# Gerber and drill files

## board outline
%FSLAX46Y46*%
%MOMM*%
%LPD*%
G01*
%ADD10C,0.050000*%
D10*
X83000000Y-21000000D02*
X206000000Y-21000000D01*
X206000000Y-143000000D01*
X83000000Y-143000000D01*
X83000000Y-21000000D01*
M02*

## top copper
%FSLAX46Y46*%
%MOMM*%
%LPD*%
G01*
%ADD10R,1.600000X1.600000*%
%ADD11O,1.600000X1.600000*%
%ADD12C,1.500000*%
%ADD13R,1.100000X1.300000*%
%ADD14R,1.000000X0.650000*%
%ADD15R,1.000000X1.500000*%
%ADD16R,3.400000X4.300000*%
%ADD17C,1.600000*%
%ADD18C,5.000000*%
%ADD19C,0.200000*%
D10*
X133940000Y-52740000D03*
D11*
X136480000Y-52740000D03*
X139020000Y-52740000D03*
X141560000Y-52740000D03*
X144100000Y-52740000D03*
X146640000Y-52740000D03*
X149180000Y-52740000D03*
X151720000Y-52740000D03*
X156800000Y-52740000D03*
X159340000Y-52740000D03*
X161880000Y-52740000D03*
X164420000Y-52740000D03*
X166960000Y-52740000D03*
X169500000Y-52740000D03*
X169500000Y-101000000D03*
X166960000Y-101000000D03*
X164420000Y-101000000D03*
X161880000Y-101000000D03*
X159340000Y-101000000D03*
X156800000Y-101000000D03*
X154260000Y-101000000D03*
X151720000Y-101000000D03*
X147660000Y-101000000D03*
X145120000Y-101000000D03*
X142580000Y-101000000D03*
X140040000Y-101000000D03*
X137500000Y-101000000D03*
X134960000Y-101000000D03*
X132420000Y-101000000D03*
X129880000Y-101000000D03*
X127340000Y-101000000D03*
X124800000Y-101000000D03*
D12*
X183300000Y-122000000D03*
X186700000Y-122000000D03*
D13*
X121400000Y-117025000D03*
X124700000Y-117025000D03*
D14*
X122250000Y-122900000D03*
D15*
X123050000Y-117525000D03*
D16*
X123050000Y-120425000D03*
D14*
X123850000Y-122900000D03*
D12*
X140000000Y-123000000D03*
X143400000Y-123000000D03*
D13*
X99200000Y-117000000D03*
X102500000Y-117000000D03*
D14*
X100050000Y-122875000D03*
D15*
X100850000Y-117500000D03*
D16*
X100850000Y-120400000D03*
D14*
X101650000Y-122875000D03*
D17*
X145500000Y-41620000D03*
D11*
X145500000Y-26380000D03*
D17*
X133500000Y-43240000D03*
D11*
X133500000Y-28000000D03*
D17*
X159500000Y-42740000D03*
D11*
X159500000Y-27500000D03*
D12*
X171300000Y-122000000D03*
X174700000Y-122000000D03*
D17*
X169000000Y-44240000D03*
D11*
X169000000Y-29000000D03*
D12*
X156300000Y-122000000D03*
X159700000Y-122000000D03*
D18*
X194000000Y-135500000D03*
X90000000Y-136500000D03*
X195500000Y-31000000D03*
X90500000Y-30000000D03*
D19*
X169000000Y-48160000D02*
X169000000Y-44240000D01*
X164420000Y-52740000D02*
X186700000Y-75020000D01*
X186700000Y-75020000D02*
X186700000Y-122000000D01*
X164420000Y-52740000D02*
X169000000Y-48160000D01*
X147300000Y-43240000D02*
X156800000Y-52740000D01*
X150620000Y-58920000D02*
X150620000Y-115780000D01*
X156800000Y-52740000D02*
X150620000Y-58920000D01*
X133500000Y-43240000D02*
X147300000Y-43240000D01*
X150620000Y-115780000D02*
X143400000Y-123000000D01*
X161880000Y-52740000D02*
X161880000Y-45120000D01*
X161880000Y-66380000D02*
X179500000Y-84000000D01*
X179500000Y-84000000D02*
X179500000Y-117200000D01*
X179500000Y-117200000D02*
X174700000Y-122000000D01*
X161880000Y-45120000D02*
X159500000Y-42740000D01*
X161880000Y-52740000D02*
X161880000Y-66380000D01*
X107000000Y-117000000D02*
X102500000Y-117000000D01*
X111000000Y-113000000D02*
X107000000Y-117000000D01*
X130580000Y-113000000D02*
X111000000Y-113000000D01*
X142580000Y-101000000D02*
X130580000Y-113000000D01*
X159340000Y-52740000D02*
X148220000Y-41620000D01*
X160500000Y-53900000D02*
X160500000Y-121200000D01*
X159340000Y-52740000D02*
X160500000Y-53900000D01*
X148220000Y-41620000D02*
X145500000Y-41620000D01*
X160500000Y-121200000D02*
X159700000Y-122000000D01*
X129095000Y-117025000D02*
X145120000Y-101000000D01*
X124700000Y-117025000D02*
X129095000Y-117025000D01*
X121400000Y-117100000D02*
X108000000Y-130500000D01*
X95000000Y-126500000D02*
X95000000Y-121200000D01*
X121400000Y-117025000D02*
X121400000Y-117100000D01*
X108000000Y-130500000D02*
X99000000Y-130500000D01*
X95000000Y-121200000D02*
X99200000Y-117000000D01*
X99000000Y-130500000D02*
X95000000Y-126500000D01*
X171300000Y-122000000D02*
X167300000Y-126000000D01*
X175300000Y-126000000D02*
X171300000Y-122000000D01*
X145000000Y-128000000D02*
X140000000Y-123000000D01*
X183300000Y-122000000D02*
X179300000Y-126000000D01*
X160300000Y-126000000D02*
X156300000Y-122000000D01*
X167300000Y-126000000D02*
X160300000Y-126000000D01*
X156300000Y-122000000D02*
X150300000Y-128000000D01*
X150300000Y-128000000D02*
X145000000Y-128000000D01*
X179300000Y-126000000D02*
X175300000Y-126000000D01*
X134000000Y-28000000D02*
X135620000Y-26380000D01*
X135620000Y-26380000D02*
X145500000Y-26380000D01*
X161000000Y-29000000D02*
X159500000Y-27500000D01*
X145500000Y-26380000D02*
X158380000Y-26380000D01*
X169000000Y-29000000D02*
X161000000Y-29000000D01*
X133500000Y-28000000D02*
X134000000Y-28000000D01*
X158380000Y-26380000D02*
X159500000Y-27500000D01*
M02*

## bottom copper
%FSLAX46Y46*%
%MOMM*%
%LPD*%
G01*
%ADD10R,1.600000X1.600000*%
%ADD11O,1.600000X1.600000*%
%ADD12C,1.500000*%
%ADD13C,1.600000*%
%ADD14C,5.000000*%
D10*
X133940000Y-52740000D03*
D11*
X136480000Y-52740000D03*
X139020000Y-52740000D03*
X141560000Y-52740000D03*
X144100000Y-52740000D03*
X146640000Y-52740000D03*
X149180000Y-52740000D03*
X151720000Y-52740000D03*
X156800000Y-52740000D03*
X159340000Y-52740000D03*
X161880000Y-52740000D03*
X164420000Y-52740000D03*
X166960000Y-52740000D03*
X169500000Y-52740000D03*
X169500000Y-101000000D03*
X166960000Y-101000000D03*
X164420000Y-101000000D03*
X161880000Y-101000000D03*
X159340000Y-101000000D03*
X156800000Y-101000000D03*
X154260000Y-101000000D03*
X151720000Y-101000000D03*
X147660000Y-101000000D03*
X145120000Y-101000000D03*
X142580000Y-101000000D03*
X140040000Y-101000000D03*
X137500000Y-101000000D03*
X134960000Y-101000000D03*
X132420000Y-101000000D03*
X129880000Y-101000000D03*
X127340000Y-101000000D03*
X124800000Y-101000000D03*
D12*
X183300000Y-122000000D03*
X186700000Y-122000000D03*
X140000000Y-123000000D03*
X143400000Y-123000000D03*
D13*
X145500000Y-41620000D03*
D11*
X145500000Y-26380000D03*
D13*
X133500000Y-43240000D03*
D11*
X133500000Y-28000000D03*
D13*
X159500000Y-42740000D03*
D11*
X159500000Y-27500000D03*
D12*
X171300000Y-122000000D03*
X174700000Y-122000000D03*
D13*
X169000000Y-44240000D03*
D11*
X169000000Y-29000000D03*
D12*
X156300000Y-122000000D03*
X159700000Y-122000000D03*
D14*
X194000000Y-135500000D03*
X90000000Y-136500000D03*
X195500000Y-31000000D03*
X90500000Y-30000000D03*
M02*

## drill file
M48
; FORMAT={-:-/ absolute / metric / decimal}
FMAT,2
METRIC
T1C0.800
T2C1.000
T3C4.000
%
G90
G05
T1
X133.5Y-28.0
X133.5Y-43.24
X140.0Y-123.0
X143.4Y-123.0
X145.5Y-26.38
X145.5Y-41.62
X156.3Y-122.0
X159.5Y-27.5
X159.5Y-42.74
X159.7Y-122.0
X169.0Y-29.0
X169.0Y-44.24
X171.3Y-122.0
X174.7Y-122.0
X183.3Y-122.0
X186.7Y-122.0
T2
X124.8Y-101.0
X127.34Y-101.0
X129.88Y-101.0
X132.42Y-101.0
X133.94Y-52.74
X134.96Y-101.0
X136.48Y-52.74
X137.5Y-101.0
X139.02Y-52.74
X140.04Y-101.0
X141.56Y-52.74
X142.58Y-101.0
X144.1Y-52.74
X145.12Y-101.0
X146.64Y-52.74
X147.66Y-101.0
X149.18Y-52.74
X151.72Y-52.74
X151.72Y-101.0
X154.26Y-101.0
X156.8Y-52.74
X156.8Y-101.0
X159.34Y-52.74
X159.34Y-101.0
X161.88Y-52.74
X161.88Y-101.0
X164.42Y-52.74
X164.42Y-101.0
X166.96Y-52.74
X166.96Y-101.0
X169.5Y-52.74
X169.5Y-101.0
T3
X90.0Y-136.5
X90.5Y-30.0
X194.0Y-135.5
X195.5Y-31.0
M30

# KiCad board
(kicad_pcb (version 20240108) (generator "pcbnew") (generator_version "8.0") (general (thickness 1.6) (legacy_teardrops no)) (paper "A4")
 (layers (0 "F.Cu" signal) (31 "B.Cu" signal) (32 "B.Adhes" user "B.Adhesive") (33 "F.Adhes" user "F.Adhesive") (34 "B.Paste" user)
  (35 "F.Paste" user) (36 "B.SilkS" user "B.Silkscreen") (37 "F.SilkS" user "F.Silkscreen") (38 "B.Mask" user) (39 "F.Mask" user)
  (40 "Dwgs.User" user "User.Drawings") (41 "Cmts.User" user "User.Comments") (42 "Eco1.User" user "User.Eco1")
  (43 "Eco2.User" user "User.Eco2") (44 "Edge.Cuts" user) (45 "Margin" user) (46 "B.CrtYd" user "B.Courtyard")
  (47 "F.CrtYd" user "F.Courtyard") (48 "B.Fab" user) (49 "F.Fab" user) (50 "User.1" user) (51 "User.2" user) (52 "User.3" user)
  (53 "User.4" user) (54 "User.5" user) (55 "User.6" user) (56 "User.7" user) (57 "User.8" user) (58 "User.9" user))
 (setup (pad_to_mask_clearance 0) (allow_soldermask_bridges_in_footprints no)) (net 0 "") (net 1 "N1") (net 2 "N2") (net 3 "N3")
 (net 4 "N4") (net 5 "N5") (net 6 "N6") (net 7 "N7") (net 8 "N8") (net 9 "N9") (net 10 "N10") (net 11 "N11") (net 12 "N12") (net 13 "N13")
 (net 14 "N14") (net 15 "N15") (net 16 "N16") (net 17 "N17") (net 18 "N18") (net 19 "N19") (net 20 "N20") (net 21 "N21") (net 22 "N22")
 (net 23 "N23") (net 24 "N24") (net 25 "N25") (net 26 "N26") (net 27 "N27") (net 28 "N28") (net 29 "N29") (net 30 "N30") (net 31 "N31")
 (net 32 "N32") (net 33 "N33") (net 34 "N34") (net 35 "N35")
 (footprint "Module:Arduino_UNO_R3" (layer "F.Cu") (at 133.94 52.74)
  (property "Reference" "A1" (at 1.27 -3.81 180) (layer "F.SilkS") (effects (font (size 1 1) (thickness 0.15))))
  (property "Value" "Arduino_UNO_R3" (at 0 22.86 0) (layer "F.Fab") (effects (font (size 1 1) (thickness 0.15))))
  (pad "1" thru_hole rect (at 0 0 90) (size 1.6 1.6) (drill 1) (layers "*.Cu" "*.Mask") (remove_unused_layers no) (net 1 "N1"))
  (pad "2" thru_hole oval (at 2.54 0 90) (size 1.6 1.6) (drill 1) (layers "*.Cu" "*.Mask") (remove_unused_layers no) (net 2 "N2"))
  (pad "3" thru_hole oval (at 5.08 0 90) (size 1.6 1.6) (drill 1) (layers "*.Cu" "*.Mask") (remove_unused_layers no) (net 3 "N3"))
  (pad "4" thru_hole oval (at 7.62 0 90) (size 1.6 1.6) (drill 1) (layers "*.Cu" "*.Mask") (remove_unused_layers no) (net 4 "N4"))
  (pad "5" thru_hole oval (at 10.16 0 90) (size 1.6 1.6) (drill 1) (layers "*.Cu" "*.Mask") (remove_unused_layers no) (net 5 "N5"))
  (pad "6" thru_hole oval (at 12.7 0 90) (size 1.6 1.6) (drill 1) (layers "*.Cu" "*.Mask") (remove_unused_layers no) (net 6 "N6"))
  (pad "7" thru_hole oval (at 15.24 0 90) (size 1.6 1.6) (drill 1) (layers "*.Cu" "*.Mask") (remove_unused_layers no) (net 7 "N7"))
  (pad "8" thru_hole oval (at 17.78 0 90) (size 1.6 1.6) (drill 1) (layers "*.Cu" "*.Mask") (remove_unused_layers no) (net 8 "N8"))
  (pad "9" thru_hole oval (at 22.86 0 90) (size 1.6 1.6) (drill 1) (layers "*.Cu" "*.Mask") (remove_unused_layers no) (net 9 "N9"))
  (pad "10" thru_hole oval (at 25.4 0 90) (size 1.6 1.6) (drill 1) (layers "*.Cu" "*.Mask") (remove_unused_layers no) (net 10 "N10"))
  (pad "11" thru_hole oval (at 27.94 0 90) (size 1.6 1.6) (drill 1) (layers "*.Cu" "*.Mask") (remove_unused_layers no) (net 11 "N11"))
  (pad "12" thru_hole oval (at 30.48 0 90) (size 1.6 1.6) (drill 1) (layers "*.Cu" "*.Mask") (remove_unused_layers no) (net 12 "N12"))
  (pad "13" thru_hole oval (at 33.02 0 90) (size 1.6 1.6) (drill 1) (layers "*.Cu" "*.Mask") (remove_unused_layers no) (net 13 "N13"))
  (pad "14" thru_hole oval (at 35.56 0 90) (size 1.6 1.6) (drill 1) (layers "*.Cu" "*.Mask") (remove_unused_layers no) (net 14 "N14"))
  (pad "15" thru_hole oval (at 35.56 48.26 90) (size 1.6 1.6) (drill 1) (layers "*.Cu" "*.Mask") (remove_unused_layers no) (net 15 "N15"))
  (pad "16" thru_hole oval (at 33.02 48.26 90) (size 1.6 1.6) (drill 1) (layers "*.Cu" "*.Mask") (remove_unused_layers no) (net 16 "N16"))
  (pad "17" thru_hole oval (at 30.48 48.26 90) (size 1.6 1.6) (drill 1) (layers "*.Cu" "*.Mask") (remove_unused_layers no) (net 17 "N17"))
  (pad "18" thru_hole oval (at 27.94 48.26 90) (size 1.6 1.6) (drill 1) (layers "*.Cu" "*.Mask") (remove_unused_layers no) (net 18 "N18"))
  (pad "19" thru_hole oval (at 25.4 48.26 90) (size 1.6 1.6) (drill 1) (layers "*.Cu" "*.Mask") (remove_unused_layers no) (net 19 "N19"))
  (pad "20" thru_hole oval (at 22.86 48.26 90) (size 1.6 1.6) (drill 1) (layers "*.Cu" "*.Mask") (remove_unused_layers no) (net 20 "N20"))
  (pad "21" thru_hole oval (at 20.32 48.26 90) (size 1.6 1.6) (drill 1) (layers "*.Cu" "*.Mask") (remove_unused_layers no) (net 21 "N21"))
  (pad "22" thru_hole oval (at 17.78 48.26 90) (size 1.6 1.6) (drill 1) (layers "*.Cu" "*.Mask") (remove_unused_layers no) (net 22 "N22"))
  (pad "23" thru_hole oval (at 13.72 48.26 90) (size 1.6 1.6) (drill 1) (layers "*.Cu" "*.Mask") (remove_unused_layers no) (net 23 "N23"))
  (pad "24" thru_hole oval (at 11.18 48.26 90) (size 1.6 1.6) (drill 1) (layers "*.Cu" "*.Mask") (remove_unused_layers no) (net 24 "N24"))
  (pad "25" thru_hole oval (at 8.64 48.26 90) (size 1.6 1.6) (drill 1) (layers "*.Cu" "*.Mask") (remove_unused_layers no) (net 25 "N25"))
  (pad "26" thru_hole oval (at 6.1 48.26 90) (size 1.6 1.6) (drill 1) (layers "*.Cu" "*.Mask") (remove_unused_layers no) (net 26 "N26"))
  (pad "27" thru_hole oval (at 3.56 48.26 90) (size 1.6 1.6) (drill 1) (layers "*.Cu" "*.Mask") (remove_unused_layers no) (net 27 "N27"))
  (pad "28" thru_hole oval (at 1.02 48.26 90) (size 1.6 1.6) (drill 1) (layers "*.Cu" "*.Mask") (remove_unused_layers no) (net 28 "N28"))
  (pad "29" thru_hole oval (at -1.52 48.26 90) (size 1.6 1.6) (drill 1) (layers "*.Cu" "*.Mask") (remove_unused_layers no) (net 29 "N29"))
  (pad "30" thru_hole oval (at -4.06 48.26 90) (size 1.6 1.6) (drill 1) (layers "*.Cu" "*.Mask") (remove_unused_layers no) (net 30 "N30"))
  (pad "31" thru_hole oval (at -6.6 48.26 90) (size 1.6 1.6) (drill 1) (layers "*.Cu" "*.Mask") (remove_unused_layers no) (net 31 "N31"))
  (pad "32" thru_hole oval (at -9.14 48.26 90) (size 1.6 1.6) (drill 1) (layers "*.Cu" "*.Mask") (remove_unused_layers no) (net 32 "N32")))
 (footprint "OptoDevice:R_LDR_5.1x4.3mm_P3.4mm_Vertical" (layer "F.Cu") (at 183.3 122)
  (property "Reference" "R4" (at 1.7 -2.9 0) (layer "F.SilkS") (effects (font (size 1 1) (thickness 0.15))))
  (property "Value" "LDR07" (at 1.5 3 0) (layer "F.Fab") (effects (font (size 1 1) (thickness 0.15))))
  (pad "1" thru_hole circle (at 0 0) (size 1.5 1.5) (drill 0.8) (layers "*.Cu" "*.Mask") (remove_unused_layers no) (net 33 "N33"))
  (pad "2" thru_hole circle (at 3.4 0) (size 1.5 1.5) (drill 0.8) (layers "*.Cu" "*.Mask") (remove_unused_layers no) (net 12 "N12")))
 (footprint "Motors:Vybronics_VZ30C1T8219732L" (layer "F.Cu") (at 123.05 121.375)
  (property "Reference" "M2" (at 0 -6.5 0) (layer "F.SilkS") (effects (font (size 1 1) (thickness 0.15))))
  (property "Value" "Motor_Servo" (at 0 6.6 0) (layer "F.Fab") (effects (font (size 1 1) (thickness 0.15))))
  (pad "" smd rect (at -0.85 -2.315 270) (size 1.07 1.4) (layers "F.Paste"))
  (pad "" smd rect (at -0.85 -0.905 270) (size 1.07 1.4) (layers "F.Paste"))
  (pad "" smd rect (at -0.85 0.505 270) (size 1.07 1.4) (layers "F.Paste"))
  (pad "" smd rect (at 0.85 -2.315 270) (size 1.07 1.4) (layers "F.Paste"))
  (pad "" smd rect (at 0.85 -0.905 270) (size 1.07 1.4) (layers "F.Paste"))
  (pad "" smd rect (at 0.85 0.505 270) (size 1.07 1.4) (layers "F.Paste"))
  (pad "1" smd rect (at -1.65 -4.35 270) (size 1.3 1.1) (layers "F.Cu" "F.Paste" "F.Mask") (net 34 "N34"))
  (pad "2" smd rect (at 1.65 -4.35 270) (size 1.3 1.1) (layers "F.Cu" "F.Paste" "F.Mask") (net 24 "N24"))
  (pad "SH" smd rect (at -0.8 1.525) (size 1 0.65) (layers "F.Cu" "F.Paste" "F.Mask"))
  (pad "SH" smd rect (at 0 -3.85 270) (size 1.5 1) (layers "F.Cu" "F.Paste" "F.Mask"))
  (pad "SH" smd rect (at 0 -0.95 270) (size 4.3 3.4) (layers "F.Cu" "F.Mask"))
  (pad "SH" smd rect (at 0.8 1.525) (size 1 0.65) (layers "F.Cu" "F.Paste" "F.Mask")))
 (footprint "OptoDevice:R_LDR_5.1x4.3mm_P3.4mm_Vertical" (layer "F.Cu") (at 140 123)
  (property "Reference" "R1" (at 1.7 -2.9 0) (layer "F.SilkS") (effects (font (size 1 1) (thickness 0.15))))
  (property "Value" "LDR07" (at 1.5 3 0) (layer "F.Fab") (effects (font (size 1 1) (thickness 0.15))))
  (pad "1" thru_hole circle (at 0 0) (size 1.5 1.5) (drill 0.8) (layers "*.Cu" "*.Mask") (remove_unused_layers no) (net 33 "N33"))
  (pad "2" thru_hole circle (at 3.4 0) (size 1.5 1.5) (drill 0.8) (layers "*.Cu" "*.Mask") (remove_unused_layers no) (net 9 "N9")))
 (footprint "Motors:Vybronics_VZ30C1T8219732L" (layer "F.Cu") (at 100.85 121.35)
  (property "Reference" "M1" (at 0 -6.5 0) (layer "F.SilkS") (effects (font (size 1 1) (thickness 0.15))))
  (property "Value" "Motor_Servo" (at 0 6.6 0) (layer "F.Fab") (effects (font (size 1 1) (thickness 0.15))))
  (pad "" smd rect (at -0.85 -2.315 270) (size 1.07 1.4) (layers "F.Paste"))
  (pad "" smd rect (at -0.85 -0.905 270) (size 1.07 1.4) (layers "F.Paste"))
  (pad "" smd rect (at -0.85 0.505 270) (size 1.07 1.4) (layers "F.Paste"))
  (pad "" smd rect (at 0.85 -2.315 270) (size 1.07 1.4) (layers "F.Paste"))
  (pad "" smd rect (at 0.85 -0.905 270) (size 1.07 1.4) (layers "F.Paste"))
  (pad "" smd rect (at 0.85 0.505 270) (size 1.07 1.4) (layers "F.Paste"))
  (pad "1" smd rect (at -1.65 -4.35 270) (size 1.3 1.1) (layers "F.Cu" "F.Paste" "F.Mask") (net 34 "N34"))
  (pad "2" smd rect (at 1.65 -4.35 270) (size 1.3 1.1) (layers "F.Cu" "F.Paste" "F.Mask") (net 25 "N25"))
  (pad "SH" smd rect (at -0.8 1.525) (size 1 0.65) (layers "F.Cu" "F.Paste" "F.Mask"))
  (pad "SH" smd rect (at 0 -3.85 270) (size 1.5 1) (layers "F.Cu" "F.Paste" "F.Mask"))
  (pad "SH" smd rect (at 0 -0.95 270) (size 4.3 3.4) (layers "F.Cu" "F.Mask"))
  (pad "SH" smd rect (at 0.8 1.525) (size 1 0.65) (layers "F.Cu" "F.Paste" "F.Mask")))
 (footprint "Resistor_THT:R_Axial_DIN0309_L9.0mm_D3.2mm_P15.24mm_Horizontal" (layer "F.Cu") (at 145.5 41.62 90)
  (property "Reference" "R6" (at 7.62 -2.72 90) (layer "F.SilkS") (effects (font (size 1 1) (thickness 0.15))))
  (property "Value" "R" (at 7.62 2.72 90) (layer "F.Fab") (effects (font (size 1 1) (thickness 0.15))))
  (pad "1" thru_hole circle (at 0 0 90) (size 1.6 1.6) (drill 0.8) (layers "*.Cu" "*.Mask") (remove_unused_layers no) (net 10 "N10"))
  (pad "2" thru_hole oval (at 15.24 0 90) (size 1.6 1.6) (drill 0.8) (layers "*.Cu" "*.Mask") (remove_unused_layers no) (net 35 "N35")))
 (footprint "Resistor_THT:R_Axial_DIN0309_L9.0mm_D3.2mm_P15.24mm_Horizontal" (layer "F.Cu") (at 133.5 43.24 90)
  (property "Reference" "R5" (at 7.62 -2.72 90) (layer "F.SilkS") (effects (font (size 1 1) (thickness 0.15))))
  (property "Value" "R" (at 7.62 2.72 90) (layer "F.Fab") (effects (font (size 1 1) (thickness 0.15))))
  (pad "1" thru_hole circle (at 0 0 90) (size 1.6 1.6) (drill 0.8) (layers "*.Cu" "*.Mask") (remove_unused_layers no) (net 9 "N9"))
  (pad "2" thru_hole oval (at 15.24 0 90) (size 1.6 1.6) (drill 0.8) (layers "*.Cu" "*.Mask") (remove_unused_layers no) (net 35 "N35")))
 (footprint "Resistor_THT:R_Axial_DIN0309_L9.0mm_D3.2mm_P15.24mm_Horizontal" (layer "F.Cu") (at 159.5 42.74 90)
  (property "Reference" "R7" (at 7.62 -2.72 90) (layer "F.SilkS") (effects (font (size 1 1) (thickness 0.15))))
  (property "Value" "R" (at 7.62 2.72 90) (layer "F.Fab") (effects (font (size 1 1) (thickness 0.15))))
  (pad "1" thru_hole circle (at 0 0 90) (size 1.6 1.6) (drill 0.8) (layers "*.Cu" "*.Mask") (remove_unused_layers no) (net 11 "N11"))
  (pad "2" thru_hole oval (at 15.24 0 90) (size 1.6 1.6) (drill 0.8) (layers "*.Cu" "*.Mask") (remove_unused_layers no) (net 35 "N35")))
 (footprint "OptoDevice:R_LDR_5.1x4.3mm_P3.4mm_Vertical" (layer "F.Cu") (at 171.3 122)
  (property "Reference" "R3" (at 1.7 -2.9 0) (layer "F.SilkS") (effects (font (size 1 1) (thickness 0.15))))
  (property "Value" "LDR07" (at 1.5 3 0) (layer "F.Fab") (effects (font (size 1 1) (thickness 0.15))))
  (pad "1" thru_hole circle (at 0 0) (size 1.5 1.5) (drill 0.8) (layers "*.Cu" "*.Mask") (remove_unused_layers no) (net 33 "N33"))
  (pad "2" thru_hole circle (at 3.4 0) (size 1.5 1.5) (drill 0.8) (layers "*.Cu" "*.Mask") (remove_unused_layers no) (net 11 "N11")))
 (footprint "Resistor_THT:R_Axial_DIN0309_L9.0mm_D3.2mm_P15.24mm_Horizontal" (layer "F.Cu") (at 169 44.24 90)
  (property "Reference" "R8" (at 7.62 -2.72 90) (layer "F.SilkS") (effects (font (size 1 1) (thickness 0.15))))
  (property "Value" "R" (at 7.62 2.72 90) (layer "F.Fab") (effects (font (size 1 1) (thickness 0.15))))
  (pad "1" thru_hole circle (at 0 0 90) (size 1.6 1.6) (drill 0.8) (layers "*.Cu" "*.Mask") (remove_unused_layers no) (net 12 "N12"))
  (pad "2" thru_hole oval (at 15.24 0 90) (size 1.6 1.6) (drill 0.8) (layers "*.Cu" "*.Mask") (remove_unused_layers no) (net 35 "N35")))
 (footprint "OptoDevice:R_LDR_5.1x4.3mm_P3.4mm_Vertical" (layer "F.Cu") (at 156.3 122)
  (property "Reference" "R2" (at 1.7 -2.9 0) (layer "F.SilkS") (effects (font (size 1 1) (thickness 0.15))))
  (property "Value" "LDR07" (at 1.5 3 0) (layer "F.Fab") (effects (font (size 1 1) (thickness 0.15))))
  (pad "1" thru_hole circle (at 0 0) (size 1.5 1.5) (drill 0.8) (layers "*.Cu" "*.Mask") (remove_unused_layers no) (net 33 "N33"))
  (pad "2" thru_hole circle (at 3.4 0) (size 1.5 1.5) (drill 0.8) (layers "*.Cu" "*.Mask") (remove_unused_layers no) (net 10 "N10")))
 (gr_rect (start 83 21) (end 206 143) (stroke (width 0.05) (type default)) (fill none) (layer "Edge.Cuts"))
 (via (at 194 135.5) (size 5) (drill 4) (layers "F.Cu" "B.Cu") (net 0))
 (via (at 90 136.5) (size 5) (drill 4) (layers "F.Cu" "B.Cu") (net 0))
 (via (at 195.5 31) (size 5) (drill 4) (layers "F.Cu" "B.Cu") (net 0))
 (via (at 90.5 30) (size 5) (drill 4) (layers "F.Cu" "B.Cu") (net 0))
 (segment (start 169 48.16) (end 169 44.24) (width 0.2) (layer "F.Cu") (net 12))
 (segment (start 164.42 52.74) (end 186.7 75.02) (width 0.2) (layer "F.Cu") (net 12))
 (segment (start 186.7 75.02) (end 186.7 122) (width 0.2) (layer "F.Cu") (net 12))
 (segment (start 164.42 52.74) (end 169 48.16) (width 0.2) (layer "F.Cu") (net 12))
 (segment (start 147.3 43.24) (end 156.8 52.74) (width 0.2) (layer "F.Cu") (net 9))
 (segment (start 150.62 58.92) (end 150.62 115.78) (width 0.2) (layer "F.Cu") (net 9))
 (segment (start 156.8 52.74) (end 150.62 58.92) (width 0.2) (layer "F.Cu") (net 9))
 (segment (start 133.5 43.24) (end 147.3 43.24) (width 0.2) (layer "F.Cu") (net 9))
 (segment (start 150.62 115.78) (end 143.4 123) (width 0.2) (layer "F.Cu") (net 9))
 (segment (start 161.88 52.74) (end 161.88 45.12) (width 0.2) (layer "F.Cu") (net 11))
 (segment (start 161.88 66.38) (end 179.5 84) (width 0.2) (layer "F.Cu") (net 11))
 (segment (start 179.5 84) (end 179.5 117.2) (width 0.2) (layer "F.Cu") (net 11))
 (segment (start 179.5 117.2) (end 174.7 122) (width 0.2) (layer "F.Cu") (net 11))
 (segment (start 161.88 45.12) (end 159.5 42.74) (width 0.2) (layer "F.Cu") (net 11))
 (segment (start 161.88 52.74) (end 161.88 66.38) (width 0.2) (layer "F.Cu") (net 11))
 (segment (start 107 117) (end 102.5 117) (width 0.2) (layer "F.Cu") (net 25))
 (segment (start 111 113) (end 107 117) (width 0.2) (layer "F.Cu") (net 25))
 (segment (start 130.58 113) (end 111 113) (width 0.2) (layer "F.Cu") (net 25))
 (segment (start 142.58 101) (end 130.58 113) (width 0.2) (layer "F.Cu") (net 25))
 (segment (start 159.34 52.74) (end 148.22 41.62) (width 0.2) (layer "F.Cu") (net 10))
 (segment (start 160.5 53.9) (end 160.5 121.2) (width 0.2) (layer "F.Cu") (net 10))
 (segment (start 159.34 52.74) (end 160.5 53.9) (width 0.2) (layer "F.Cu") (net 10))
 (segment (start 148.22 41.62) (end 145.5 41.62) (width 0.2) (layer "F.Cu") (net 10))
 (segment (start 160.5 121.2) (end 159.7 122) (width 0.2) (layer "F.Cu") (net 10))
 (segment (start 129.095 117.025) (end 145.12 101) (width 0.2) (layer "F.Cu") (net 24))
 (segment (start 124.7 117.025) (end 129.095 117.025) (width 0.2) (layer "F.Cu") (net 24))
 (segment (start 121.4 117.1) (end 108 130.5) (width 0.2) (layer "F.Cu") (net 34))
 (segment (start 95 126.5) (end 95 121.2) (width 0.2) (layer "F.Cu") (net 34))
 (segment (start 121.4 117.025) (end 121.4 117.1) (width 0.2) (layer "F.Cu") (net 34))
 (segment (start 108 130.5) (end 99 130.5) (width 0.2) (layer "F.Cu") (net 34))
 (segment (start 95 121.2) (end 99.2 117) (width 0.2) (layer "F.Cu") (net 34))
 (segment (start 99 130.5) (end 95 126.5) (width 0.2) (layer "F.Cu") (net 34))
 (segment (start 171.3 122) (end 167.3 126) (width 0.2) (layer "F.Cu") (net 33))
 (segment (start 175.3 126) (end 171.3 122) (width 0.2) (layer "F.Cu") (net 33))
 (segment (start 145 128) (end 140 123) (width 0.2) (layer "F.Cu") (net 33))
 (segment (start 183.3 122) (end 179.3 126) (width 0.2) (layer "F.Cu") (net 33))
 (segment (start 160.3 126) (end 156.3 122) (width 0.2) (layer "F.Cu") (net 33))
 (segment (start 167.3 126) (end 160.3 126) (width 0.2) (layer "F.Cu") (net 33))
 (segment (start 156.3 122) (end 150.3 128) (width 0.2) (layer "F.Cu") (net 33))
 (segment (start 150.3 128) (end 145 128) (width 0.2) (layer "F.Cu") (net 33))
 (segment (start 179.3 126) (end 175.3 126) (width 0.2) (layer "F.Cu") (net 33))
 (segment (start 134 28) (end 135.62 26.38) (width 0.2) (layer "F.Cu") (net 35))
 (segment (start 135.62 26.38) (end 145.5 26.38) (width 0.2) (layer "F.Cu") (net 35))
 (segment (start 161 29) (end 159.5 27.5) (width 0.2) (layer "F.Cu") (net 35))
 (segment (start 145.5 26.38) (end 158.38 26.38) (width 0.2) (layer "F.Cu") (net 35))
 (segment (start 169 29) (end 161 29) (width 0.2) (layer "F.Cu") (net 35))
 (segment (start 133.5 28) (end 134 28) (width 0.2) (layer "F.Cu") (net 35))
 (segment (start 158.38 26.38) (end 159.5 27.5) (width 0.2) (layer "F.Cu") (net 35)))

